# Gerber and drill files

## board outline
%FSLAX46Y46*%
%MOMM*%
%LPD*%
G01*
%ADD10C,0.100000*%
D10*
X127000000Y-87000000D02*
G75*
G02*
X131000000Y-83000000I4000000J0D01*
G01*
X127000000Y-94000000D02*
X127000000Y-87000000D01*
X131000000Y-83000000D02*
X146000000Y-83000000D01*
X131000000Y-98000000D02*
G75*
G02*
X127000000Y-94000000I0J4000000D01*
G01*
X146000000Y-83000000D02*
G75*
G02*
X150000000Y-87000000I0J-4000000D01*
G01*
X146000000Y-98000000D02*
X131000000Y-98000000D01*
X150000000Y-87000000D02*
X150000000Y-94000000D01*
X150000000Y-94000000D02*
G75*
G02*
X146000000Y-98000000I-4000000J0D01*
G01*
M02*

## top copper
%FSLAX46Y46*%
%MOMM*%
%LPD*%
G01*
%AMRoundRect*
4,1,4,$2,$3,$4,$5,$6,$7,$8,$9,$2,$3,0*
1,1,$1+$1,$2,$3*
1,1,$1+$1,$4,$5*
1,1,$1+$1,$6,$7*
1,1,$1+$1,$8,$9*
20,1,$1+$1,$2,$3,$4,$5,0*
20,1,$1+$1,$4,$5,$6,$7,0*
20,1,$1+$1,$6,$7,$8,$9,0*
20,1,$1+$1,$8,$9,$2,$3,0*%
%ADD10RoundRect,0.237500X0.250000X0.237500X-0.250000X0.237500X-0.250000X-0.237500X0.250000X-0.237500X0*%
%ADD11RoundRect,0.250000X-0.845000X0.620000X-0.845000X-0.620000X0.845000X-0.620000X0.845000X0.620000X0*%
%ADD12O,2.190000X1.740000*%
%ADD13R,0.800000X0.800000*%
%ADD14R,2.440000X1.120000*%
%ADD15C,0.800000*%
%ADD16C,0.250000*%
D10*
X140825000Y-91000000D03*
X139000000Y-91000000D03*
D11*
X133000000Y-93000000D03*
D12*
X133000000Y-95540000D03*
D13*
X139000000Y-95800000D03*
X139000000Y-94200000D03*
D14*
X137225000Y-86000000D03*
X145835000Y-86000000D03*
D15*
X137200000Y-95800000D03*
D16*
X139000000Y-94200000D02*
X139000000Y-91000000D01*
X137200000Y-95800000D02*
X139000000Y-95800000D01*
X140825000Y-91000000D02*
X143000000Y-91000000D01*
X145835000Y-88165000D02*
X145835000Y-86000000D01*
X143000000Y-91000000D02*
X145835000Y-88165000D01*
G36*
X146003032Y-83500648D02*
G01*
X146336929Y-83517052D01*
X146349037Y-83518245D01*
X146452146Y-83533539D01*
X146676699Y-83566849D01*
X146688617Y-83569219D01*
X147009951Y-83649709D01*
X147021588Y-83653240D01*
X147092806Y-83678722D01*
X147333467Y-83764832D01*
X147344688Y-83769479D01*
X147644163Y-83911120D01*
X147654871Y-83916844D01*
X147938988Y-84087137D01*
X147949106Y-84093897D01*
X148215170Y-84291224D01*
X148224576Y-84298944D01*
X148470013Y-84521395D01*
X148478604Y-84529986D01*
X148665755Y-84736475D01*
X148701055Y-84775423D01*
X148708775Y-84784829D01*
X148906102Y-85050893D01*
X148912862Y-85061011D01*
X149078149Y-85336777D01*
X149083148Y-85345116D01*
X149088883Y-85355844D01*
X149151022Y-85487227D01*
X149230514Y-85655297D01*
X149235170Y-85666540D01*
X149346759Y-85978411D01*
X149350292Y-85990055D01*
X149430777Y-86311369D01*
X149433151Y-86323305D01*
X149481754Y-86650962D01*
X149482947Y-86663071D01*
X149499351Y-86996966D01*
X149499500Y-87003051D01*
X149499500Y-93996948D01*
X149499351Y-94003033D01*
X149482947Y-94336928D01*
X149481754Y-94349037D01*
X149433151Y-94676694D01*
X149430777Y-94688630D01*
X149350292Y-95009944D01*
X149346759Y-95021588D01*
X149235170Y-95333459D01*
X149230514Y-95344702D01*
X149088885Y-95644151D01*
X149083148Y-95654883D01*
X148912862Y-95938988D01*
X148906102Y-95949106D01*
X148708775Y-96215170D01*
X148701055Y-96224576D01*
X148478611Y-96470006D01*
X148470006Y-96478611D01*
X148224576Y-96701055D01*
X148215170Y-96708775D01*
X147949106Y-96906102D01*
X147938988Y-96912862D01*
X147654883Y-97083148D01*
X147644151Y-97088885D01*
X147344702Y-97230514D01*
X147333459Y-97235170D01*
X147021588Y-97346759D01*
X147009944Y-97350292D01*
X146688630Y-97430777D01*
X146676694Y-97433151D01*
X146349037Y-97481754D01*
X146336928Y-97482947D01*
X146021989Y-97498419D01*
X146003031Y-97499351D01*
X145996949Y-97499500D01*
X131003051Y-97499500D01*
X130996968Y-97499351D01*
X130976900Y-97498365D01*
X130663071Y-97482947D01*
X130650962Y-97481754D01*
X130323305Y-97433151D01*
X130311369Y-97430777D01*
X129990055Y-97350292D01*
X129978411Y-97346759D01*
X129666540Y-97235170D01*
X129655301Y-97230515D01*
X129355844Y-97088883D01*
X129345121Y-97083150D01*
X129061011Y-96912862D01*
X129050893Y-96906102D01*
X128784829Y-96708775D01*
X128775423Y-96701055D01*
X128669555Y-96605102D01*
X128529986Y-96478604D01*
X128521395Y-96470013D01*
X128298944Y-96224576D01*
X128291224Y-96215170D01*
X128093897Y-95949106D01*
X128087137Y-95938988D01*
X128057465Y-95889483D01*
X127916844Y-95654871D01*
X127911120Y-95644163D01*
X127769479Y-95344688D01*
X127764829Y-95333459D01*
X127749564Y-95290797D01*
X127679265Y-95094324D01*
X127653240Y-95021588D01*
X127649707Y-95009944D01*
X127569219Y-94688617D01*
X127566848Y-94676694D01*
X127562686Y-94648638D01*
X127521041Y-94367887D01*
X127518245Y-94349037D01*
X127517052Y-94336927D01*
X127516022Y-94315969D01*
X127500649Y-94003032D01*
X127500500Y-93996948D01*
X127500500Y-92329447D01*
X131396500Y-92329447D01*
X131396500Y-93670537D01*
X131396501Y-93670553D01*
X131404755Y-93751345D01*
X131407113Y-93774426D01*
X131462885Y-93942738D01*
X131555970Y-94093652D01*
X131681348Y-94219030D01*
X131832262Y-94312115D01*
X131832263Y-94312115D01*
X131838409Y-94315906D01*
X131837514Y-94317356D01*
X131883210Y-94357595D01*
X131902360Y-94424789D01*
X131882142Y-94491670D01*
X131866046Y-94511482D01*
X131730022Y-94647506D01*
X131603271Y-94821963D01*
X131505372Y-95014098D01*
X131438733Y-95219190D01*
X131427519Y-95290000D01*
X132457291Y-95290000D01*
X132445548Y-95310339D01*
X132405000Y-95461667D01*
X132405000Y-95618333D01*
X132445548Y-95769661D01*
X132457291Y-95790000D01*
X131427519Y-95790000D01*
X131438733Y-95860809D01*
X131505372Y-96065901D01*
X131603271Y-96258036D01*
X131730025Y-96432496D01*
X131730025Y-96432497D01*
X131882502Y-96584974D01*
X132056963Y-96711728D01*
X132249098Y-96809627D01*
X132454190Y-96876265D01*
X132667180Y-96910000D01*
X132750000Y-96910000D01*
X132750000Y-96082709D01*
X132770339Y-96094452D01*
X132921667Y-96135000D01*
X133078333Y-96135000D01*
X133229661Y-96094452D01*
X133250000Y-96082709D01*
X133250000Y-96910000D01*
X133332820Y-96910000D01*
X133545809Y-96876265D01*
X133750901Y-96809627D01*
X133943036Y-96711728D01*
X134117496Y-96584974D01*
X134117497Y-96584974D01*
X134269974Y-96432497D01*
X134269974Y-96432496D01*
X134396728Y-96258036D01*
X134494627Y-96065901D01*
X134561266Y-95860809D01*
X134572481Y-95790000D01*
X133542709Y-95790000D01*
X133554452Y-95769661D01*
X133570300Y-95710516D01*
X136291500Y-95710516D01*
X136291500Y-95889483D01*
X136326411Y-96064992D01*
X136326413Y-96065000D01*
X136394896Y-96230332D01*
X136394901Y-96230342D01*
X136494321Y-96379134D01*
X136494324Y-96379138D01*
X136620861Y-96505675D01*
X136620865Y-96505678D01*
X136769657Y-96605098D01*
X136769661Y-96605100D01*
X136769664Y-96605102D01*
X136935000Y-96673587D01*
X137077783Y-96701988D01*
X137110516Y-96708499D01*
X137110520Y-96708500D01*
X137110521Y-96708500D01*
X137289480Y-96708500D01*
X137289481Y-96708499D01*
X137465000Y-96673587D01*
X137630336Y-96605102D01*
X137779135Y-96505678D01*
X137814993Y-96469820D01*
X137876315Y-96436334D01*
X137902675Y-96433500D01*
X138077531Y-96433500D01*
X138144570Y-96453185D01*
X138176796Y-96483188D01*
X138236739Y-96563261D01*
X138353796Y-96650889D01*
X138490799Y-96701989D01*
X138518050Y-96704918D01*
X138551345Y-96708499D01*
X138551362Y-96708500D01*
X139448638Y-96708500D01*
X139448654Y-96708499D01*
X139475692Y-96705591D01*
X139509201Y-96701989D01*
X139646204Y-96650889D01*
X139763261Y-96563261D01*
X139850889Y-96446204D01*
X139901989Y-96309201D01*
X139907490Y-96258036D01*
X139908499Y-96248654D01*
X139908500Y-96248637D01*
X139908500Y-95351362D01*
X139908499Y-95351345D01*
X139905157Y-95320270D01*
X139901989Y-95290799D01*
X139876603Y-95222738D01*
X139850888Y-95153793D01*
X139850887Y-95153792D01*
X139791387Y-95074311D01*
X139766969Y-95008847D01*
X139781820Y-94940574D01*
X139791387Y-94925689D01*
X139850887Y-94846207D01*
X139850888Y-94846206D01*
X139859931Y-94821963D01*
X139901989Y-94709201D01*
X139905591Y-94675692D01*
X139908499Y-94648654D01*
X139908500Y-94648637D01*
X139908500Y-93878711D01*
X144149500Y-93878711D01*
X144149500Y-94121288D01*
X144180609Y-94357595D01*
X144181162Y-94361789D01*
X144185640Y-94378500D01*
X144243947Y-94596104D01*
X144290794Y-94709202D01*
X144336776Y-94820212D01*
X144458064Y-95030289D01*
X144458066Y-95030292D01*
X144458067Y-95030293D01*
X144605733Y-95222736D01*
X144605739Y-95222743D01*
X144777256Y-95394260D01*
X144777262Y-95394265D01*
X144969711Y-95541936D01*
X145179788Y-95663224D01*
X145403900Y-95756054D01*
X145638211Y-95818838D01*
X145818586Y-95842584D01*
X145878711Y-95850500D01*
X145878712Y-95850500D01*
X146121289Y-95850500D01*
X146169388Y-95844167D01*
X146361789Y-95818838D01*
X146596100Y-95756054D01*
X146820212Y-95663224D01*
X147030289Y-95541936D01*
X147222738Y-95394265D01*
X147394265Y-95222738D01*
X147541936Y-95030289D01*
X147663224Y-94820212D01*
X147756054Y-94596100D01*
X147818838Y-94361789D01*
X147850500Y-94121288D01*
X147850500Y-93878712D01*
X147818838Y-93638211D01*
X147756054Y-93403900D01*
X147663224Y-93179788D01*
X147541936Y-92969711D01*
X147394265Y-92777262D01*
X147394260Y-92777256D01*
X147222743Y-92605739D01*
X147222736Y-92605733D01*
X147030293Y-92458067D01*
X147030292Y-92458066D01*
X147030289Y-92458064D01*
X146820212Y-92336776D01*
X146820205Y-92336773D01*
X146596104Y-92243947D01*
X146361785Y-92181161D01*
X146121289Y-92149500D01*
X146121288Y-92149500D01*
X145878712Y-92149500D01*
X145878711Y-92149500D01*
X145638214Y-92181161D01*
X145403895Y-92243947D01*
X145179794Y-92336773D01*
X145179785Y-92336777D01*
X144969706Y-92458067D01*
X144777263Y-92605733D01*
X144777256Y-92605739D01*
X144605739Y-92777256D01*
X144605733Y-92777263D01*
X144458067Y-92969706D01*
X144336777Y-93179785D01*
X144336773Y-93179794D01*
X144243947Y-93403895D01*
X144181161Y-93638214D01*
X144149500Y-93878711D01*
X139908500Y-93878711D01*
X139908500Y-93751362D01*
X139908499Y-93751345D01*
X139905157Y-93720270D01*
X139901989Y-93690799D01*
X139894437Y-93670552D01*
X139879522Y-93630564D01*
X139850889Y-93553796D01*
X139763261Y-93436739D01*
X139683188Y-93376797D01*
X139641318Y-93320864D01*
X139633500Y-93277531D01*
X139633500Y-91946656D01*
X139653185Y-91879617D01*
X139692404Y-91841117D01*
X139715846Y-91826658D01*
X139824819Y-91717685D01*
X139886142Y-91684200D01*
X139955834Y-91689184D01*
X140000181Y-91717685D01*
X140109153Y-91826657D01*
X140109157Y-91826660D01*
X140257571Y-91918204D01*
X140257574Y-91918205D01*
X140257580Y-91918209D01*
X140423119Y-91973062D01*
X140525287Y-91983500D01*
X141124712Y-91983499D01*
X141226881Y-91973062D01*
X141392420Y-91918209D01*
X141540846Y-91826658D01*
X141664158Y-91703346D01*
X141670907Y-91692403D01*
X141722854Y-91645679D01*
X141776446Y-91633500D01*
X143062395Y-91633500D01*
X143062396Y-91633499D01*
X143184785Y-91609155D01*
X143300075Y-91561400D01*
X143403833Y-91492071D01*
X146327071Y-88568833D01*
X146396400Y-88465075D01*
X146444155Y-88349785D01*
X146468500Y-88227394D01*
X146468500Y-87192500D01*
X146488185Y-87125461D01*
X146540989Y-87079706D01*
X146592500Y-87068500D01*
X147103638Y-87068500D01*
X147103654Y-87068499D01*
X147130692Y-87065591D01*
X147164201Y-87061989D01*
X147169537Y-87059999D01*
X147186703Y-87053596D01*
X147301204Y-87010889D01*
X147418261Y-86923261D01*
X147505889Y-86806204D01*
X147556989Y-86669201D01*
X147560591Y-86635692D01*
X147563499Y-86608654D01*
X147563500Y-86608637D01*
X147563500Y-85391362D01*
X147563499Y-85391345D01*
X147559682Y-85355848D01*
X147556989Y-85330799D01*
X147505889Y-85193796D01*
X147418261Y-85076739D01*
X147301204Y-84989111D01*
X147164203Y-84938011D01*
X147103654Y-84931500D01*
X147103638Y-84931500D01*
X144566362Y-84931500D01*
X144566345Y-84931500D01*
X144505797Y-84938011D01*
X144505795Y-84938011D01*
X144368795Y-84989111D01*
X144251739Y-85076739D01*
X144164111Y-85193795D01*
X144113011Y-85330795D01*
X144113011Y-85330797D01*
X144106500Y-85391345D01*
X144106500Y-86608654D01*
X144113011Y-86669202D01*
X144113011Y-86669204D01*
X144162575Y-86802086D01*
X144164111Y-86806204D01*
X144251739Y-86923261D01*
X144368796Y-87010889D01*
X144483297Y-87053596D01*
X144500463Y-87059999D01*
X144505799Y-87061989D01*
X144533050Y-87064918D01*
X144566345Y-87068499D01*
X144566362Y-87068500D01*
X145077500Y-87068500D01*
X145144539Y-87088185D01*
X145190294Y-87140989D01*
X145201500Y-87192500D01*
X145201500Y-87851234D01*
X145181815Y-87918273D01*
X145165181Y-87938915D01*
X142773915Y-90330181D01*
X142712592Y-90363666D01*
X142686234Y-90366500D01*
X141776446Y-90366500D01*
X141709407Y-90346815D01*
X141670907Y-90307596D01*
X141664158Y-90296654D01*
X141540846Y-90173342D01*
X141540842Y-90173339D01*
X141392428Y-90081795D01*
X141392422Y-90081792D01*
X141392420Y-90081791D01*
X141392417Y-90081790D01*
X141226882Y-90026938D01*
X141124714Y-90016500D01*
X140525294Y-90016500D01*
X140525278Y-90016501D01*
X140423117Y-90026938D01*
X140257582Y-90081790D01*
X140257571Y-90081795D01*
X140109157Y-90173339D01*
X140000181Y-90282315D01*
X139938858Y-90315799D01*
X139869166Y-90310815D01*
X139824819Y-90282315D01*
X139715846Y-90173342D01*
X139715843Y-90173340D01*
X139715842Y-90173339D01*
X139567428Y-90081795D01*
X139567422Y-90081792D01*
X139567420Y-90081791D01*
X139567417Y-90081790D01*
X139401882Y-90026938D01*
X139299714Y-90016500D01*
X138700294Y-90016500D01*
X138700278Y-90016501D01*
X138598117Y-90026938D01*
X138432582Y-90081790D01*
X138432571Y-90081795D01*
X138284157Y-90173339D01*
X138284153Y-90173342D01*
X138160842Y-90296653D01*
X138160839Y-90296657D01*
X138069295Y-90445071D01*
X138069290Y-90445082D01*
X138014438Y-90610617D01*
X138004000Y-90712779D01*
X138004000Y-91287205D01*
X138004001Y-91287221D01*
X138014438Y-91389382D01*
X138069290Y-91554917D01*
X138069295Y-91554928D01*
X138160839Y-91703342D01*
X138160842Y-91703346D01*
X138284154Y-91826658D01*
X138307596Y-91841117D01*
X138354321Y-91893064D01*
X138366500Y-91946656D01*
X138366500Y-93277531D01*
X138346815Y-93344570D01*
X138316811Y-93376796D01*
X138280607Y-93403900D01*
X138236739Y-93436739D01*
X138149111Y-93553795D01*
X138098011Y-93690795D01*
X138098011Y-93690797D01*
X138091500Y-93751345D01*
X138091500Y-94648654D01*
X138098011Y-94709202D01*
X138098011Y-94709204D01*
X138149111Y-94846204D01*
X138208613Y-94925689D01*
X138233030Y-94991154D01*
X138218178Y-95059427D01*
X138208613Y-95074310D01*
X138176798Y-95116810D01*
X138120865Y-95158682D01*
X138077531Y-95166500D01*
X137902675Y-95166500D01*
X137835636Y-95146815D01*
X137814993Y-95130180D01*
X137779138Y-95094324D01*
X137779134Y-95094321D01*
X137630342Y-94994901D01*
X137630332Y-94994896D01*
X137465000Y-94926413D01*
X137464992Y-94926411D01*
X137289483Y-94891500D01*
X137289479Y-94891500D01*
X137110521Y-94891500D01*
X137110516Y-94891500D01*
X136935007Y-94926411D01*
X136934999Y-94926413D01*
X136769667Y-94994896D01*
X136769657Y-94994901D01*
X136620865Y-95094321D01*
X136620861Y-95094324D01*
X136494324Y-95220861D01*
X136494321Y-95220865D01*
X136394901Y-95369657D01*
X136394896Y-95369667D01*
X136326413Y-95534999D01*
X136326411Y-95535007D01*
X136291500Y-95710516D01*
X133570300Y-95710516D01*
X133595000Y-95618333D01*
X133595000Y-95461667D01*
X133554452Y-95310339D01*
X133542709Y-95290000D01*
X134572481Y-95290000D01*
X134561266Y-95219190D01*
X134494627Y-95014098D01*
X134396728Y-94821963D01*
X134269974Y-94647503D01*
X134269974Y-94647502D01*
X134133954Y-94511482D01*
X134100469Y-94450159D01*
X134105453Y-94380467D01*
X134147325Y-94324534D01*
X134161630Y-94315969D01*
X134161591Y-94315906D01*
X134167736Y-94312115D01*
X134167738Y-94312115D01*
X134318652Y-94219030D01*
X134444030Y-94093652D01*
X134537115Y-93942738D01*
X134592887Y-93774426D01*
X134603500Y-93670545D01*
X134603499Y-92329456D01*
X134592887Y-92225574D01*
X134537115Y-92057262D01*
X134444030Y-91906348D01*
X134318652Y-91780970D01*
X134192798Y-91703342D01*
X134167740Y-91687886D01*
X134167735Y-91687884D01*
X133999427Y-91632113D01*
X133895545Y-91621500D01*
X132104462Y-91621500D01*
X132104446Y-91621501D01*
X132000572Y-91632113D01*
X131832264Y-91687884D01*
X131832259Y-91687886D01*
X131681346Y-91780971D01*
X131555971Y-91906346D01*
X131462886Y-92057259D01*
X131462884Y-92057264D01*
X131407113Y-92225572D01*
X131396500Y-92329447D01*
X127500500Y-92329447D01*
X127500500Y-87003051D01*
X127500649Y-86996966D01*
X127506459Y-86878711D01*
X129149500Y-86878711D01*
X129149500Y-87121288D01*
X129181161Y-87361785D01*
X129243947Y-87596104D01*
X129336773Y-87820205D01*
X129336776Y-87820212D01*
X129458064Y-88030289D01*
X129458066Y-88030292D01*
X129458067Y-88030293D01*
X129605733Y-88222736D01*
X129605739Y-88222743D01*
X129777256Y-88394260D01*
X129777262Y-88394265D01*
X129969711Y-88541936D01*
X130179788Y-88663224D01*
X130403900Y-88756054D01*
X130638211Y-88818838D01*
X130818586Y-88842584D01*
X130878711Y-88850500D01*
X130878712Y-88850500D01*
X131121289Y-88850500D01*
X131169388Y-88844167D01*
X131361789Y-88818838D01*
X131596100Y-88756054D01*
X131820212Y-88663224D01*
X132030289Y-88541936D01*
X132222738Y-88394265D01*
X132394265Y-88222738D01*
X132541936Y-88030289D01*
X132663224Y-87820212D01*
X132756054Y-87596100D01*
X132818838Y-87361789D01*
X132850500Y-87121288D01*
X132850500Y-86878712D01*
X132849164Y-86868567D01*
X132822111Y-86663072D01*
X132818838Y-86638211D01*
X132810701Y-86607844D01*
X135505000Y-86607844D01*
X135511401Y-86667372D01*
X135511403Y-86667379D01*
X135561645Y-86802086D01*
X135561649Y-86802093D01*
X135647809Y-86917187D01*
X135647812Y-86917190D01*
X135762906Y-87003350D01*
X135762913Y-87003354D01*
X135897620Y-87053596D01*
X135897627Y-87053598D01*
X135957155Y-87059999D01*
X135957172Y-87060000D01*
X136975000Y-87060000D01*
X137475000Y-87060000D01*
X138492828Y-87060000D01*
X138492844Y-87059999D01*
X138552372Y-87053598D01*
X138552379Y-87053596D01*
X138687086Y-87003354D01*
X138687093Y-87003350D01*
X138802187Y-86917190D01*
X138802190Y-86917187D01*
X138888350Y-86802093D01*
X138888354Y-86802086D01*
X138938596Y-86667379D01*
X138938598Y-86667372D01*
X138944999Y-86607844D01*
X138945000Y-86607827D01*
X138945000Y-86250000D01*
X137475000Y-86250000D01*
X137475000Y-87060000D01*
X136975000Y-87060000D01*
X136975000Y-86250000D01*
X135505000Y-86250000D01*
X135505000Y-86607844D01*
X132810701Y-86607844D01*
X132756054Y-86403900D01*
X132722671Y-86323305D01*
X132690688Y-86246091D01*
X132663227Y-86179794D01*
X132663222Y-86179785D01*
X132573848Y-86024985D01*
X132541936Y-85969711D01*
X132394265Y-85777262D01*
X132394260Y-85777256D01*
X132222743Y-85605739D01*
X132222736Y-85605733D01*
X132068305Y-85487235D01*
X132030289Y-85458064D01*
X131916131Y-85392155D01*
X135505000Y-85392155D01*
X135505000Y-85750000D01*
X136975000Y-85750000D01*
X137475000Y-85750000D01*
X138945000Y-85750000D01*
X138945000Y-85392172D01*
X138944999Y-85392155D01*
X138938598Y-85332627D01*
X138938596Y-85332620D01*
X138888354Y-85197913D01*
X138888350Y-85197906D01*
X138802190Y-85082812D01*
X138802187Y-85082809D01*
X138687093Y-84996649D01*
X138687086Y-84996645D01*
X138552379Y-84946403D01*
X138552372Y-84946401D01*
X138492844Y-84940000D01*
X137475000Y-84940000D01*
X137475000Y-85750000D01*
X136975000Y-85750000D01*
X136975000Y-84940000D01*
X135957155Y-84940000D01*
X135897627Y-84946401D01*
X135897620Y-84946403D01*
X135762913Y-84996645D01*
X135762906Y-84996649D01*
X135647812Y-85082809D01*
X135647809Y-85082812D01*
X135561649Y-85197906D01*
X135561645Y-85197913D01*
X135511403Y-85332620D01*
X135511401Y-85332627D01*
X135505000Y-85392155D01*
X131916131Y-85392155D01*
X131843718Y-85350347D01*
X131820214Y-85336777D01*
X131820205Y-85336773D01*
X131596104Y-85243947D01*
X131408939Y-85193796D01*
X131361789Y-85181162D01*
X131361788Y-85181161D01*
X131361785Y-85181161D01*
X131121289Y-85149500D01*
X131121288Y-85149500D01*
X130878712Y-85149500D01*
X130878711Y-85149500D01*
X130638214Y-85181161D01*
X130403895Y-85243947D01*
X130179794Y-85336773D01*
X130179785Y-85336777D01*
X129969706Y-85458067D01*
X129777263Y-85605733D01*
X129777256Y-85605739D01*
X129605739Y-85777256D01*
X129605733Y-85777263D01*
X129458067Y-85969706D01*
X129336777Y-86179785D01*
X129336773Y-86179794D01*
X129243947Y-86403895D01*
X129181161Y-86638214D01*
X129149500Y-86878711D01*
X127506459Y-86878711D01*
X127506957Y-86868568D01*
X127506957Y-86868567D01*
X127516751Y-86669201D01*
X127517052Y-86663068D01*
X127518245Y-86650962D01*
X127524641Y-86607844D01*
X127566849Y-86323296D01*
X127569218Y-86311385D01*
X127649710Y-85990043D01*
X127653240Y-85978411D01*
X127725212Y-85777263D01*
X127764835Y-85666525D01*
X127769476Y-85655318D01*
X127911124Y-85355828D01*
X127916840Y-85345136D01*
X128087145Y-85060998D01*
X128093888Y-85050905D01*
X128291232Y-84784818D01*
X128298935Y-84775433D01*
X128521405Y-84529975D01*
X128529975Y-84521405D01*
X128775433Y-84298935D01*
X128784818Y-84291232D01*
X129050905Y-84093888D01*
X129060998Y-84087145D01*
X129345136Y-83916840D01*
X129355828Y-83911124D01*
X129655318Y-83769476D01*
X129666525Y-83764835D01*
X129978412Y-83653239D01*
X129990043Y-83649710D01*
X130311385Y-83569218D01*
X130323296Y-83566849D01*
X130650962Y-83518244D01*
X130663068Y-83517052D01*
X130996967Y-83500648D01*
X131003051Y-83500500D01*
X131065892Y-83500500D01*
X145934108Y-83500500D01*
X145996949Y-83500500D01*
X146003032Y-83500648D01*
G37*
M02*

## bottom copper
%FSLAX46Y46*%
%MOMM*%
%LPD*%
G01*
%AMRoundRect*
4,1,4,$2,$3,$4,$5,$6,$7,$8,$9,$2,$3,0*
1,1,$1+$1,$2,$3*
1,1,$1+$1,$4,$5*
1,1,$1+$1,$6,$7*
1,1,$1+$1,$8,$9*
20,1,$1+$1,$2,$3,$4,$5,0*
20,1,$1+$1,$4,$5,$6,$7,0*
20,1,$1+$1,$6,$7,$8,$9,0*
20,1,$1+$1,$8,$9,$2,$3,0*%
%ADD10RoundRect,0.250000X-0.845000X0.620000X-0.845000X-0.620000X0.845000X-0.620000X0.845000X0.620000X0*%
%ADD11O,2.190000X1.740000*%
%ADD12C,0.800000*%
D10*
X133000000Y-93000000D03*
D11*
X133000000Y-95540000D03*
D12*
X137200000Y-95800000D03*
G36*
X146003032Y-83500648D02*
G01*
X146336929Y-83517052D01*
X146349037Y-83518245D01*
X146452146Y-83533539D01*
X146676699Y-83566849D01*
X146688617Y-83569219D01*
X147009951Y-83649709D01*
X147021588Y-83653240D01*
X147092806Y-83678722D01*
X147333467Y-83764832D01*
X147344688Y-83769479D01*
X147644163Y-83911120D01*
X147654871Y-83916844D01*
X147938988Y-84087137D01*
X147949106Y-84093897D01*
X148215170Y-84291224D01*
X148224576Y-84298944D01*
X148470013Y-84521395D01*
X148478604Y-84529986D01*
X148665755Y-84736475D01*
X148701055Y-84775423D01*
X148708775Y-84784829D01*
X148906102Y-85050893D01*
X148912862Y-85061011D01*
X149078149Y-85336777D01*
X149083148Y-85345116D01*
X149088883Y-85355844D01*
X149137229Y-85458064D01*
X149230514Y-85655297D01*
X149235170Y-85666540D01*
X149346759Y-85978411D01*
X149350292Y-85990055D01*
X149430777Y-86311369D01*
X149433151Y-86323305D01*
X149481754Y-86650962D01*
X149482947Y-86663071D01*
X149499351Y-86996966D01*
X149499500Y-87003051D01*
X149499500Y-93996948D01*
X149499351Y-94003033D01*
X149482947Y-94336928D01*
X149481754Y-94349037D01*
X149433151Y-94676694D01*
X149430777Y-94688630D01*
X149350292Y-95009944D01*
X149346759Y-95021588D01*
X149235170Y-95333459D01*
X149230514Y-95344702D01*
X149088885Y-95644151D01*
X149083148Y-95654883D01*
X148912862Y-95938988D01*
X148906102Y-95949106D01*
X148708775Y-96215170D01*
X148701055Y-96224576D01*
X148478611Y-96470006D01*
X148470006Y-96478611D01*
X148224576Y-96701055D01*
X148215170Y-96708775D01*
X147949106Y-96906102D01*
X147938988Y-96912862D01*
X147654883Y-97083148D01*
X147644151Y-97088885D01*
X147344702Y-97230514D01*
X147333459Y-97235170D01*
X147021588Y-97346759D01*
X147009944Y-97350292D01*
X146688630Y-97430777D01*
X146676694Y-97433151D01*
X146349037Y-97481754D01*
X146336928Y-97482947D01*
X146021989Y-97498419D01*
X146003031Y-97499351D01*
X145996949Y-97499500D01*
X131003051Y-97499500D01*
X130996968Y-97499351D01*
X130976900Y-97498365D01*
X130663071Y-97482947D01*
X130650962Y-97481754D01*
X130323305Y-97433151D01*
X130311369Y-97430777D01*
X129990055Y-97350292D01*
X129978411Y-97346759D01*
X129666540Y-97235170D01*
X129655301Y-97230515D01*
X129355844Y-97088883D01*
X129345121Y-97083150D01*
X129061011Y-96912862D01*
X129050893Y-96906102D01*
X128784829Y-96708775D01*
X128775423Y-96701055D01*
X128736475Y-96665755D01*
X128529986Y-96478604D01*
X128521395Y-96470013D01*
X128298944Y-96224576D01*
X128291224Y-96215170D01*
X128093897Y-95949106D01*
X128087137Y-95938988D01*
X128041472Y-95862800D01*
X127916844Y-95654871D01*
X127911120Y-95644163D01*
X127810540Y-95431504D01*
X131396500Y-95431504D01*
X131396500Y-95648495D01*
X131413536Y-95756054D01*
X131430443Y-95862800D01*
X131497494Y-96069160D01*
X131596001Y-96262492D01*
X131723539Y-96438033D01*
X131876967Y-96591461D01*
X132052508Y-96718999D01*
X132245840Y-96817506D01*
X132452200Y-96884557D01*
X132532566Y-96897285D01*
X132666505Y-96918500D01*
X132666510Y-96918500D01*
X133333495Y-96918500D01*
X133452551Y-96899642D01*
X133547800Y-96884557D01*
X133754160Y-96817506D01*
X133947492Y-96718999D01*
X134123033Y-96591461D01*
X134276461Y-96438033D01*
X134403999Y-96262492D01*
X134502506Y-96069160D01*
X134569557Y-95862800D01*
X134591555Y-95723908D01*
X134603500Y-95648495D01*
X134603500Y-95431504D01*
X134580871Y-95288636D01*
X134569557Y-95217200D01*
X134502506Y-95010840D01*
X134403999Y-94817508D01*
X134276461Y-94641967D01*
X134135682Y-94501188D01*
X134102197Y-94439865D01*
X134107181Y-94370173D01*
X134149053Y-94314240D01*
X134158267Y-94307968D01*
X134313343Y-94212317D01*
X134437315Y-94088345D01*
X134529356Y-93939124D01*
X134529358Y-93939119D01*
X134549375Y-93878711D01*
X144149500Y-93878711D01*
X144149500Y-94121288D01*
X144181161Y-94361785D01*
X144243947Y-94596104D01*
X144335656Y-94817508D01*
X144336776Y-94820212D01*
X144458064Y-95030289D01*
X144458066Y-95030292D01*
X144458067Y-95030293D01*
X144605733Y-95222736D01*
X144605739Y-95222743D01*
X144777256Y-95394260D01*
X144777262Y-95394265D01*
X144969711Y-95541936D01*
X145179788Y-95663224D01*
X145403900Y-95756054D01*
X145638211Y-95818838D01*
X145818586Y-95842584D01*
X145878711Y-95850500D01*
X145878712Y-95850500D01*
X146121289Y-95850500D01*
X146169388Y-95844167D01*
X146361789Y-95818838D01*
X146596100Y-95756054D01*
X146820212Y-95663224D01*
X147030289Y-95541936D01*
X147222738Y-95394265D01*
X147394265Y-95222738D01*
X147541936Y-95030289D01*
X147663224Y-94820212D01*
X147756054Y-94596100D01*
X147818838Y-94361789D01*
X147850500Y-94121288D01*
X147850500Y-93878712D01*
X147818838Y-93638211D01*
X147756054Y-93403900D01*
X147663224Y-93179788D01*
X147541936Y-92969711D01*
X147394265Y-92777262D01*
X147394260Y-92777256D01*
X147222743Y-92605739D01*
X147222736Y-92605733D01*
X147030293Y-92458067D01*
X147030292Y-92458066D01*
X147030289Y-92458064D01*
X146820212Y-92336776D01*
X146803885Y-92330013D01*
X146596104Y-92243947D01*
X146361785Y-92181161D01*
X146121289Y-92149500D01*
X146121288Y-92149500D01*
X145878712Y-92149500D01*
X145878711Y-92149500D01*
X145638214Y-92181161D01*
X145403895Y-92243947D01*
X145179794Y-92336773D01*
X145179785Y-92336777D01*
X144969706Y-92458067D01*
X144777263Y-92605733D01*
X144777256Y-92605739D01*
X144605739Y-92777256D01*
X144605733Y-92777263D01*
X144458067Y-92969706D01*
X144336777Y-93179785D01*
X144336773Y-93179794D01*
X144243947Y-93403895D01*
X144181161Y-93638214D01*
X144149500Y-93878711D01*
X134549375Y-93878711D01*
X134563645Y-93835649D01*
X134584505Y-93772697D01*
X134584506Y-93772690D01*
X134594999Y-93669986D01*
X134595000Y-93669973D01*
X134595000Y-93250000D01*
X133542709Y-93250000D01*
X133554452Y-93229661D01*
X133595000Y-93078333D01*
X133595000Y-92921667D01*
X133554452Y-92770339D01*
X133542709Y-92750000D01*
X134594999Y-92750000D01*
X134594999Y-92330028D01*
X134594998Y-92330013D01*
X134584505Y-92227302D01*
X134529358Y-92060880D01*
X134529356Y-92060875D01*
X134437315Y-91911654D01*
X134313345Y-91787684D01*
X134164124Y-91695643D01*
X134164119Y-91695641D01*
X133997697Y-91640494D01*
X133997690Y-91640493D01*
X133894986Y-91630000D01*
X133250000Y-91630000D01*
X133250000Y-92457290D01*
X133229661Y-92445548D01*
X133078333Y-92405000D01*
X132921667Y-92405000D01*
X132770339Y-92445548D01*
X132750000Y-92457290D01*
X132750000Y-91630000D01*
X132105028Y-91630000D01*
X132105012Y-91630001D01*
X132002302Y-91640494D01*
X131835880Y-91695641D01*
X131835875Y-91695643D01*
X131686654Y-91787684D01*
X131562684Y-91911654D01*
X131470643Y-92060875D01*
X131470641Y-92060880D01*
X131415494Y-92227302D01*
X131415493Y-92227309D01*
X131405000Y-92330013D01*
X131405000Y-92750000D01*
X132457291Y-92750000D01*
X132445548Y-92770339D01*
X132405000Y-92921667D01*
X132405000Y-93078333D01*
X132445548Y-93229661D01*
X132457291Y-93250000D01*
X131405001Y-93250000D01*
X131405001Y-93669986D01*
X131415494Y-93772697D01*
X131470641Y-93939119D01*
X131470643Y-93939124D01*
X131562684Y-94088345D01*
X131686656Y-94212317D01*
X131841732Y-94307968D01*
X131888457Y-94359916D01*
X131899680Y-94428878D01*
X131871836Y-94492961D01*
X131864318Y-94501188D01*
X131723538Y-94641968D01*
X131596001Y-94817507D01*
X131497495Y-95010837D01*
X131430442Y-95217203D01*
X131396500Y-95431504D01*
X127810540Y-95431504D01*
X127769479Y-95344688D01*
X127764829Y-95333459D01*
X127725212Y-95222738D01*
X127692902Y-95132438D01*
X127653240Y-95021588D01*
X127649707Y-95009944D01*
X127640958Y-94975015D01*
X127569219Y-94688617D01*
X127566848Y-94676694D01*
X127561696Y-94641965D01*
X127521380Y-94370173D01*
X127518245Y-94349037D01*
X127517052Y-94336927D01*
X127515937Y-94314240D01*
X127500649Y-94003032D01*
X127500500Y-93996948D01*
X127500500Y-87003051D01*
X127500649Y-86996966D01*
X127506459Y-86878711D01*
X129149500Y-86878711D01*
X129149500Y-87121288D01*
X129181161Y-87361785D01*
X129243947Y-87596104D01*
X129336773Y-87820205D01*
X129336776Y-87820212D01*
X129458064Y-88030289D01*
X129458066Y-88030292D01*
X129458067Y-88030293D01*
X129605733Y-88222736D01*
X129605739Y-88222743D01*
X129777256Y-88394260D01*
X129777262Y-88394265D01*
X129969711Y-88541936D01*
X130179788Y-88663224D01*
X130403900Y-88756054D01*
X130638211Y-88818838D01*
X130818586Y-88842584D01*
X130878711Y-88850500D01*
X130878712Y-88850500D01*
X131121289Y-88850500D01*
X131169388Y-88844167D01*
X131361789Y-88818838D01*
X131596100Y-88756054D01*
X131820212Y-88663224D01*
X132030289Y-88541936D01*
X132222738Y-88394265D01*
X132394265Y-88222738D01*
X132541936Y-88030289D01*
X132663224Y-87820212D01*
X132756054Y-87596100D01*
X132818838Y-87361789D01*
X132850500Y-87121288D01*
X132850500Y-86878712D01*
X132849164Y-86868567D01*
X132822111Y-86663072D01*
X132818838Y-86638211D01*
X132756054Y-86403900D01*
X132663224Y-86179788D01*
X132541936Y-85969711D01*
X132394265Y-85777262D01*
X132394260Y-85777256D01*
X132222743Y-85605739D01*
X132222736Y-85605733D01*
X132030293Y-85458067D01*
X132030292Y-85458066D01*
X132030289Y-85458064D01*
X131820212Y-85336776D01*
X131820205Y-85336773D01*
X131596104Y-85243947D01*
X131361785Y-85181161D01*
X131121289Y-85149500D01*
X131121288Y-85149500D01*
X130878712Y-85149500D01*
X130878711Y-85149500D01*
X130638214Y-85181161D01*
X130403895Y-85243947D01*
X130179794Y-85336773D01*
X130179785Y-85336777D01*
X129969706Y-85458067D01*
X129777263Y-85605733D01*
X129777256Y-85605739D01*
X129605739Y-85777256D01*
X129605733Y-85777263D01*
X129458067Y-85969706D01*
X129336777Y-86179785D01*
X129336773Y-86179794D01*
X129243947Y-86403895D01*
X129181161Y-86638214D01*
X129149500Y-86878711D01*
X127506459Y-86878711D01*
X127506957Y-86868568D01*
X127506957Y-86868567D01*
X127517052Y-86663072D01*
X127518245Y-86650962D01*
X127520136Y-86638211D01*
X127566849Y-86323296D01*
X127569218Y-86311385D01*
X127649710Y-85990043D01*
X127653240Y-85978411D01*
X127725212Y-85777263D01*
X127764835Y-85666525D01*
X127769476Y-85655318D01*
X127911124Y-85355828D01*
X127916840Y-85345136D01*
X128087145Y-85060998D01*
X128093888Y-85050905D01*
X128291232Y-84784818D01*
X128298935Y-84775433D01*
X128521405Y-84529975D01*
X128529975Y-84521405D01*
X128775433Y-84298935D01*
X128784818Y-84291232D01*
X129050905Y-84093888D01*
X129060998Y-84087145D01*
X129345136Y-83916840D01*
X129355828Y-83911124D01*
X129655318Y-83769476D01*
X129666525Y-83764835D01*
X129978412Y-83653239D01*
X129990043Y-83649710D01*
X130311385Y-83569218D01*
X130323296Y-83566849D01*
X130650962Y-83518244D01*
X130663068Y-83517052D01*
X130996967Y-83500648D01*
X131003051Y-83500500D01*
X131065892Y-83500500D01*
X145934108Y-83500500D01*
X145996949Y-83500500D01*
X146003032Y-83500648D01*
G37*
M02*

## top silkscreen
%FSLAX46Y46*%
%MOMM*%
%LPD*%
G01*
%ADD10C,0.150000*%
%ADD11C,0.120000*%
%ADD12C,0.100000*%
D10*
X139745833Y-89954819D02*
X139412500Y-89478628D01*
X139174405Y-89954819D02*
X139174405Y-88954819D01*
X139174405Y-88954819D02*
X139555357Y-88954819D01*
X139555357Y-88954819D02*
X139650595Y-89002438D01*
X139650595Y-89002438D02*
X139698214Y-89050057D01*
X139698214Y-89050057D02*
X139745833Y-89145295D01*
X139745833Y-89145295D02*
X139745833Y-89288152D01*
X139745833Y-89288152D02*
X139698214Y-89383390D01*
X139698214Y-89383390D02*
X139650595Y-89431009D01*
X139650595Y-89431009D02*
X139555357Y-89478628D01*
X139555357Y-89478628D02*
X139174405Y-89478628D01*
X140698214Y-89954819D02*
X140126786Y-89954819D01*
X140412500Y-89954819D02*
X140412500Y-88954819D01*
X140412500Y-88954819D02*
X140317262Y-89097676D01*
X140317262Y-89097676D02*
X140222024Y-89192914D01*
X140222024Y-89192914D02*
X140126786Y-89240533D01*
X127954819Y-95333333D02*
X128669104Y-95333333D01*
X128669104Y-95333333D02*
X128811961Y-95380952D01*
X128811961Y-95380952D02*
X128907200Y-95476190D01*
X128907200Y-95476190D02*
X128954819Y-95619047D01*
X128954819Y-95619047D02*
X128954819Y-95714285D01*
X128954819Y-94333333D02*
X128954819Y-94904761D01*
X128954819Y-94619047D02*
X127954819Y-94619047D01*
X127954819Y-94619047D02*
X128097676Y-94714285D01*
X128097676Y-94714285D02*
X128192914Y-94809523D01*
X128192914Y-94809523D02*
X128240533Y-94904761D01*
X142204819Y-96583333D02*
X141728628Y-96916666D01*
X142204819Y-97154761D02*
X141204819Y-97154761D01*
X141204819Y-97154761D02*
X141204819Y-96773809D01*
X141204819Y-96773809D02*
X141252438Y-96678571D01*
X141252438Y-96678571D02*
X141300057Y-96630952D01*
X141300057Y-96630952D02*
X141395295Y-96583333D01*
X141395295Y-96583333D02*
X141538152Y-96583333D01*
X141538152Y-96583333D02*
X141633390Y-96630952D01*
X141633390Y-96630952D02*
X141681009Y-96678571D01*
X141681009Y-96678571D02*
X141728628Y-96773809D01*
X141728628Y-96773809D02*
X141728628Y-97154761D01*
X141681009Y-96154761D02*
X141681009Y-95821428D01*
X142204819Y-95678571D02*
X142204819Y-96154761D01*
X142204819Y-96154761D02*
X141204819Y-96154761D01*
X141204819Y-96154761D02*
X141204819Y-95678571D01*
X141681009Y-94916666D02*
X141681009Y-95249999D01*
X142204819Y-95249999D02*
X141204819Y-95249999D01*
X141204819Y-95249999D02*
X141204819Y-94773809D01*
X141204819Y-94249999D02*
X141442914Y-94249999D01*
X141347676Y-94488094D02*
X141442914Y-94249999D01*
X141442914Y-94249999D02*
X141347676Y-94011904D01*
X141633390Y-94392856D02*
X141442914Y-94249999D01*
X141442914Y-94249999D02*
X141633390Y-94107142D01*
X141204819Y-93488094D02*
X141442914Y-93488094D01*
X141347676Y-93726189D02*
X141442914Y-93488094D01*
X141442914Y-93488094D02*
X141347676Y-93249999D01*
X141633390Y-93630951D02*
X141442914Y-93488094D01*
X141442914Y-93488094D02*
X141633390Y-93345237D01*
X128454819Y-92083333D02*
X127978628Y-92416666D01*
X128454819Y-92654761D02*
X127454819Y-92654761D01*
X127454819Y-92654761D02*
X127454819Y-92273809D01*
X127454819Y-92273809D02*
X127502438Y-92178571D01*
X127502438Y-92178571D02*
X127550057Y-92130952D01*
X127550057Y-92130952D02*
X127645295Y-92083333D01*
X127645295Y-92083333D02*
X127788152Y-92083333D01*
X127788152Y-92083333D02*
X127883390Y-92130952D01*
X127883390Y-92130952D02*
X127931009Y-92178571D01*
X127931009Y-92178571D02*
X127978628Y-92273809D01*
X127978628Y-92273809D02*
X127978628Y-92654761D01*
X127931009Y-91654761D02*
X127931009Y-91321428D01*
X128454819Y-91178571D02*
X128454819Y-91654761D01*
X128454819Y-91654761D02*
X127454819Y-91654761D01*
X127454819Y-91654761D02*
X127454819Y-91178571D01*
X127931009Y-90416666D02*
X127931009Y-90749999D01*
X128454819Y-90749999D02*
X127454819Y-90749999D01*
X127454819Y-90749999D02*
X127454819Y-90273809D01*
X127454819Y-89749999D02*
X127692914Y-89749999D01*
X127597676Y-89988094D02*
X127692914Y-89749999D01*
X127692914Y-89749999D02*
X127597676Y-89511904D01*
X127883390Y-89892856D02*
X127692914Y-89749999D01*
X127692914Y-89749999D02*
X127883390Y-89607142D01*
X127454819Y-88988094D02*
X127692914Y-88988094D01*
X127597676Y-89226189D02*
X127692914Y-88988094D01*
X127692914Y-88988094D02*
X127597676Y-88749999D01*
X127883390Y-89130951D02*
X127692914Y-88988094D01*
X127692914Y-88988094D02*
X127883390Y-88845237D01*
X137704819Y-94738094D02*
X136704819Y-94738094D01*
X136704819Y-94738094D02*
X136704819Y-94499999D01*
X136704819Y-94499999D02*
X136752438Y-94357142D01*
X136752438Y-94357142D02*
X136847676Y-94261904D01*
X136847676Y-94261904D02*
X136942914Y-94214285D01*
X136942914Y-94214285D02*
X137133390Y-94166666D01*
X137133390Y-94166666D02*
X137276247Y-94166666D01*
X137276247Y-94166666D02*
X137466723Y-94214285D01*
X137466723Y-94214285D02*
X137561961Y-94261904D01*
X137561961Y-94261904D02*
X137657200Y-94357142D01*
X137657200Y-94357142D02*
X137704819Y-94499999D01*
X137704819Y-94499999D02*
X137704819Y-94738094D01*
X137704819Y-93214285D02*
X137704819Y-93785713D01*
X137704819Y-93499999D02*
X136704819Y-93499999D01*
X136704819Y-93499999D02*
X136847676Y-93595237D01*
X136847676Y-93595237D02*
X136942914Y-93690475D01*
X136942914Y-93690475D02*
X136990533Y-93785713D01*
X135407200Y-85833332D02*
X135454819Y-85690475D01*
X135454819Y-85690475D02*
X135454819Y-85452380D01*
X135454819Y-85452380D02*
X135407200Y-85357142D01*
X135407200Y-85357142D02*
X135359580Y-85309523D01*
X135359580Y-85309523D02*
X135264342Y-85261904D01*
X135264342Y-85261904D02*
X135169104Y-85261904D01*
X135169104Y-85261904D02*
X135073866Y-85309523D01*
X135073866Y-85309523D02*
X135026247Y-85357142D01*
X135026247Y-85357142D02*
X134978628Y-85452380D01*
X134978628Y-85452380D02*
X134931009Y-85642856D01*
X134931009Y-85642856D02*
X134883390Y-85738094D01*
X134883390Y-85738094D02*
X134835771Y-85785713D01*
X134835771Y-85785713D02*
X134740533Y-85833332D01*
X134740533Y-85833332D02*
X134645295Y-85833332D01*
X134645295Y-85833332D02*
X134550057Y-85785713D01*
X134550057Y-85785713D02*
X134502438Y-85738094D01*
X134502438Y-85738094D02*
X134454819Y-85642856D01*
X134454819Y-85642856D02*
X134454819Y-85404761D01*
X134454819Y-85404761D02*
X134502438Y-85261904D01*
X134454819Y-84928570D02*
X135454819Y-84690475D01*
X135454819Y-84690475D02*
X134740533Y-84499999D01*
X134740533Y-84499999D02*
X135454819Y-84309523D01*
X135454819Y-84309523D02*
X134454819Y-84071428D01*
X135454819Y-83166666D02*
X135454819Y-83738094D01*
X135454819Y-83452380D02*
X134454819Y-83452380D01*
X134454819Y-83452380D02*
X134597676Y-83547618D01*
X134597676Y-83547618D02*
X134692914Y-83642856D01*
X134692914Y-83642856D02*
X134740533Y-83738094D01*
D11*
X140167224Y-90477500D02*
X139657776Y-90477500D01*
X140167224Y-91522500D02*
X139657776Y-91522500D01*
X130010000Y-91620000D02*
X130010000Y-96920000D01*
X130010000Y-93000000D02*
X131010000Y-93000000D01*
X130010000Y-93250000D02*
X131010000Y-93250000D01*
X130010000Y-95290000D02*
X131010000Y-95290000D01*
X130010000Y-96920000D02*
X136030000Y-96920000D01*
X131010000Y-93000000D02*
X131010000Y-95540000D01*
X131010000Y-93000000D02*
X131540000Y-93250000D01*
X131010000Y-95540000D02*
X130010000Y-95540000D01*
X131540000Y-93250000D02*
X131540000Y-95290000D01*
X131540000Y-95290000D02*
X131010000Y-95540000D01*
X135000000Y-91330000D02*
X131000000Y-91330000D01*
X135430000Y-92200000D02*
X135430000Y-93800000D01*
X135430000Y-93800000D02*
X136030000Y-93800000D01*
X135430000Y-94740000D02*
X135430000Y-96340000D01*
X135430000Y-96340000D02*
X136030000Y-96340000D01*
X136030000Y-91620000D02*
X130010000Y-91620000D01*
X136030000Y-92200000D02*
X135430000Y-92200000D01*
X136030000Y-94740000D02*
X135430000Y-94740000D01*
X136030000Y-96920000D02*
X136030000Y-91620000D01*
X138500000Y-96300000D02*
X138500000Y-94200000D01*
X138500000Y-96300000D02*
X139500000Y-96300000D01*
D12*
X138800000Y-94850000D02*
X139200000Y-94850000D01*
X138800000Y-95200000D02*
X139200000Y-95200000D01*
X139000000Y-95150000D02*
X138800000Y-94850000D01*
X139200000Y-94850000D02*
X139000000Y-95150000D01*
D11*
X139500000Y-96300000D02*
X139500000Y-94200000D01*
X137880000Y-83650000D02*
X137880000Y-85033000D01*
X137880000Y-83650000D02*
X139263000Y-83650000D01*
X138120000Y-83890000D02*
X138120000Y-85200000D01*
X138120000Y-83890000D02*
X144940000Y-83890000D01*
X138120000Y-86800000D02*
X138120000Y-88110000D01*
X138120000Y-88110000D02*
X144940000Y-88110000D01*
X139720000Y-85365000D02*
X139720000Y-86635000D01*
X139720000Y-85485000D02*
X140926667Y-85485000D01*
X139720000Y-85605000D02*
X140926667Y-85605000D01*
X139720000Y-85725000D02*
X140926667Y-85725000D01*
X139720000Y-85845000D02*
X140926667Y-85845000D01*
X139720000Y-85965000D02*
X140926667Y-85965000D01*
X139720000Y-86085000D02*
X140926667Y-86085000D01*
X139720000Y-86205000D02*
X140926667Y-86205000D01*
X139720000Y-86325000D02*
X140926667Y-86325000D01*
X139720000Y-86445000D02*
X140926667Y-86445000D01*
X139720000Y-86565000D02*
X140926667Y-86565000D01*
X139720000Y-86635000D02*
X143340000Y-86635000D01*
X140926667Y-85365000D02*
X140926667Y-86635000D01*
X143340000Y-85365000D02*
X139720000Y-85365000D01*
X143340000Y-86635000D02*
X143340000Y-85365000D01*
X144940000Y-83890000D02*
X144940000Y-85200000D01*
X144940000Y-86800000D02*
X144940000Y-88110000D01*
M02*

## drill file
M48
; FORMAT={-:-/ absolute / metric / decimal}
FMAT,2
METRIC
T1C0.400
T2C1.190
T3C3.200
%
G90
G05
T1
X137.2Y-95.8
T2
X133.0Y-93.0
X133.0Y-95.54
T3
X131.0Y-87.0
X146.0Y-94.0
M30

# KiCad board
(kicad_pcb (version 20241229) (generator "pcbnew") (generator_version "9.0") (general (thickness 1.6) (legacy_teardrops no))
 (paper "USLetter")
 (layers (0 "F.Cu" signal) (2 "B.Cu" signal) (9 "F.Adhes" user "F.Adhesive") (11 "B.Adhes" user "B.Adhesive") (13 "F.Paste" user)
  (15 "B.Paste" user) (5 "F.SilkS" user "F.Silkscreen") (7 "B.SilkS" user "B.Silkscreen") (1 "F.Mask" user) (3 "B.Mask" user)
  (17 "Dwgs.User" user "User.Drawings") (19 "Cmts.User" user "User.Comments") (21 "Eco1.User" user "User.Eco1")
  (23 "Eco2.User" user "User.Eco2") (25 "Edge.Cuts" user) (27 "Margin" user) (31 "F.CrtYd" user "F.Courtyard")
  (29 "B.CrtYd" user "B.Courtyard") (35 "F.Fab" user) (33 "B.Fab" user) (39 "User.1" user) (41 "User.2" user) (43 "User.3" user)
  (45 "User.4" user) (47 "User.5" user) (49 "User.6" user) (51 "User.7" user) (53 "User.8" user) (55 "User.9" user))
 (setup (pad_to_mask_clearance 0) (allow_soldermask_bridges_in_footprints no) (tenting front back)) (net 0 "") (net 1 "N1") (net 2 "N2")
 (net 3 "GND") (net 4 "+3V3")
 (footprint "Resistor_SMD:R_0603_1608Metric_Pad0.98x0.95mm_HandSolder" (layer "F.Cu") (at 139.9125 91 180)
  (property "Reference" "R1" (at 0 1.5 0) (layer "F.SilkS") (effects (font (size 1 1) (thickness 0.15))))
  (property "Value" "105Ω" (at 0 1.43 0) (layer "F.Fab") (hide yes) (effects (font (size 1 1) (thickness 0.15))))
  (fp_line (start -0.254724 0.5225) (end 0.254724 0.5225) (stroke (width 0.12) (type solid)) (layer "F.SilkS"))
  (fp_line (start -0.254724 -0.5225) (end 0.254724 -0.5225) (stroke (width 0.12) (type solid)) (layer "F.SilkS"))
  (pad "1" smd roundrect (at -0.9125 0 180) (size 0.975 0.95) (layers "F.Cu" "F.Mask" "F.Paste") (roundrect_rratio 0.25) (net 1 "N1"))
  (pad "2" smd roundrect (at 0.9125 0 180) (size 0.975 0.95) (layers "F.Cu" "F.Mask" "F.Paste") (roundrect_rratio 0.25) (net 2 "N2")))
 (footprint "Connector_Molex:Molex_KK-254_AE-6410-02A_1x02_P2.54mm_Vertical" (layer "F.Cu") (at 133 93 -90)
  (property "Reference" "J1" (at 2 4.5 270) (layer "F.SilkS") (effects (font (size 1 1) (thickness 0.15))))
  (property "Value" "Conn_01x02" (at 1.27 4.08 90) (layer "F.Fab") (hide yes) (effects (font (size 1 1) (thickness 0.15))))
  (fp_line (start -1.38 2.99) (end 3.92 2.99) (stroke (width 0.12) (type solid)) (layer "F.SilkS"))
  (fp_line (start 0 2.99) (end 0 1.99) (stroke (width 0.12) (type solid)) (layer "F.SilkS"))
  (fp_line (start 0.25 2.99) (end 0.25 1.99) (stroke (width 0.12) (type solid)) (layer "F.SilkS"))
  (fp_line (start 2.29 2.99) (end 2.29 1.99) (stroke (width 0.12) (type solid)) (layer "F.SilkS"))
  (fp_line (start 3.92 2.99) (end 3.92 -3.03) (stroke (width 0.12) (type solid)) (layer "F.SilkS"))
  (fp_line (start 0 1.99) (end 2.54 1.99) (stroke (width 0.12) (type solid)) (layer "F.SilkS"))
  (fp_line (start 0 1.99) (end 0.25 1.46) (stroke (width 0.12) (type solid)) (layer "F.SilkS"))
  (fp_line (start 2.54 1.99) (end 2.54 2.99) (stroke (width 0.12) (type solid)) (layer "F.SilkS"))
  (fp_line (start 0.25 1.46) (end 2.29 1.46) (stroke (width 0.12) (type solid)) (layer "F.SilkS"))
  (fp_line (start 2.29 1.46) (end 2.54 1.99) (stroke (width 0.12) (type solid)) (layer "F.SilkS"))
  (fp_line (start -1.67 -2) (end -1.67 2) (stroke (width 0.12) (type solid)) (layer "F.SilkS"))
  (fp_line (start -0.8 -2.43) (end 0.8 -2.43) (stroke (width 0.12) (type solid)) (layer "F.SilkS"))
  (fp_line (start 0.8 -2.43) (end 0.8 -3.03) (stroke (width 0.12) (type solid)) (layer "F.SilkS"))
  (fp_line (start 1.74 -2.43) (end 3.34 -2.43) (stroke (width 0.12) (type solid)) (layer "F.SilkS"))
  (fp_line (start 3.34 -2.43) (end 3.34 -3.03) (stroke (width 0.12) (type solid)) (layer "F.SilkS"))
  (fp_line (start -1.38 -3.03) (end -1.38 2.99) (stroke (width 0.12) (type solid)) (layer "F.SilkS"))
  (fp_line (start -0.8 -3.03) (end -0.8 -2.43) (stroke (width 0.12) (type solid)) (layer "F.SilkS"))
  (fp_line (start 1.74 -3.03) (end 1.74 -2.43) (stroke (width 0.12) (type solid)) (layer "F.SilkS"))
  (fp_line (start 3.92 -3.03) (end -1.38 -3.03) (stroke (width 0.12) (type solid)) (layer "F.SilkS"))
  (pad "1" thru_hole roundrect (at 0 0 270) (size 1.74 2.19) (drill 1.19) (layers "*.Cu" "*.Mask") (remove_unused_layers no)
   (roundrect_rratio 0.143678) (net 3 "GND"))
  (pad "2" thru_hole oval (at 2.54 0 270) (size 1.74 2.19) (drill 1.19) (layers "*.Cu" "*.Mask") (remove_unused_layers no) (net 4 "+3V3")))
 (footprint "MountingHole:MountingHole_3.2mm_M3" (layer "F.Cu") (at 146 94)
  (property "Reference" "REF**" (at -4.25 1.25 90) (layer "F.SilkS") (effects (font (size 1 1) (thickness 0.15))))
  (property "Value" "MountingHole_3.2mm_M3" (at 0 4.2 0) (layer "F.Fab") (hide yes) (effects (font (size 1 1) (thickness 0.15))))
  (pad "" np_thru_hole circle (at 0 0) (size 3.2 3.2) (drill 3.2) (layers "*.Cu" "*.Mask")))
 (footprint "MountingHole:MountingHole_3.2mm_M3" (layer "F.Cu") (at 131 87)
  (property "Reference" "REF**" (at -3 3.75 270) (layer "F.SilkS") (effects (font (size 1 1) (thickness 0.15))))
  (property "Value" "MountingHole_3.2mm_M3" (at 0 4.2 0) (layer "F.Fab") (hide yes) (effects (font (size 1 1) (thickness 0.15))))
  (pad "" np_thru_hole circle (at 0 0) (size 3.2 3.2) (drill 3.2) (layers "*.Cu" "*.Mask")))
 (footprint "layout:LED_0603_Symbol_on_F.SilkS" (layer "F.Cu") (at 139 95 90)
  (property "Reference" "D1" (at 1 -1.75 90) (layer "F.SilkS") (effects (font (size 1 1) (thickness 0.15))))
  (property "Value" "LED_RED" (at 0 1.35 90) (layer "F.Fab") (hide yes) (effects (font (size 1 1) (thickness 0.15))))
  (fp_line (start -1.3 -0.5) (end 0.8 -0.5) (stroke (width 0.12) (type solid)) (layer "F.SilkS"))
  (fp_line (start -1.3 -0.5) (end -1.3 0.5) (stroke (width 0.12) (type solid)) (layer "F.SilkS"))
  (fp_line (start 0.15 -0.2) (end 0.15 0.2) (stroke (width 0.1) (type solid)) (layer "F.SilkS"))
  (fp_line (start -0.2 -0.2) (end -0.2 0.2) (stroke (width 0.1) (type solid)) (layer "F.SilkS"))
  (fp_line (start -0.15 0) (end 0.15 -0.2) (stroke (width 0.1) (type solid)) (layer "F.SilkS"))
  (fp_line (start 0.15 0.2) (end -0.15 0) (stroke (width 0.1) (type solid)) (layer "F.SilkS"))
  (fp_line (start -1.3 0.5) (end 0.8 0.5) (stroke (width 0.12) (type solid)) (layer "F.SilkS"))
  (pad "1" smd rect (at -0.8 0 270) (size 0.8 0.8) (layers "F.Cu" "F.Mask" "F.Paste") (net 3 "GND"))
  (pad "2" smd rect (at 0.8 0 270) (size 0.8 0.8) (layers "F.Cu" "F.Mask" "F.Paste") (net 2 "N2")))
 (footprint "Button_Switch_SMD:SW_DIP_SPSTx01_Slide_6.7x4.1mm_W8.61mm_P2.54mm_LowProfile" (layer "F.Cu") (at 141.53 86)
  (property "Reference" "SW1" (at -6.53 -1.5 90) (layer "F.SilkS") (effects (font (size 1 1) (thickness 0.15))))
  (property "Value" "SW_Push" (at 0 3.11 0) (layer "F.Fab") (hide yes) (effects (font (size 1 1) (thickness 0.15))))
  (fp_line (start -3.65 -2.35) (end -3.65 -0.967) (stroke (width 0.12) (type solid)) (layer "F.SilkS"))
  (fp_line (start -3.65 -2.35) (end -2.267 -2.35) (stroke (width 0.12) (type solid)) (layer "F.SilkS"))
  (fp_line (start -3.41 -2.11) (end -3.41 -0.8) (stroke (width 0.12) (type solid)) (layer "F.SilkS"))
  (fp_line (start -3.41 -2.11) (end 3.41 -2.11) (stroke (width 0.12) (type solid)) (layer "F.SilkS"))
  (fp_line (start -3.41 0.8) (end -3.41 2.11) (stroke (width 0.12) (type solid)) (layer "F.SilkS"))
  (fp_line (start -3.41 2.11) (end 3.41 2.11) (stroke (width 0.12) (type solid)) (layer "F.SilkS"))
  (fp_line (start -1.81 -0.635) (end -1.81 0.635) (stroke (width 0.12) (type solid)) (layer "F.SilkS"))
  (fp_line (start -1.81 -0.515) (end -0.603333 -0.515) (stroke (width 0.12) (type solid)) (layer "F.SilkS"))
  (fp_line (start -1.81 -0.395) (end -0.603333 -0.395) (stroke (width 0.12) (type solid)) (layer "F.SilkS"))
  (fp_line (start -1.81 -0.275) (end -0.603333 -0.275) (stroke (width 0.12) (type solid)) (layer "F.SilkS"))
  (fp_line (start -1.81 -0.155) (end -0.603333 -0.155) (stroke (width 0.12) (type solid)) (layer "F.SilkS"))
  (fp_line (start -1.81 -0.035) (end -0.603333 -0.035) (stroke (width 0.12) (type solid)) (layer "F.SilkS"))
  (fp_line (start -1.81 0.085) (end -0.603333 0.085) (stroke (width 0.12) (type solid)) (layer "F.SilkS"))
  (fp_line (start -1.81 0.205) (end -0.603333 0.205) (stroke (width 0.12) (type solid)) (layer "F.SilkS"))
  (fp_line (start -1.81 0.325) (end -0.603333 0.325) (stroke (width 0.12) (type solid)) (layer "F.SilkS"))
  (fp_line (start -1.81 0.445) (end -0.603333 0.445) (stroke (width 0.12) (type solid)) (layer "F.SilkS"))
  (fp_line (start -1.81 0.565) (end -0.603333 0.565) (stroke (width 0.12) (type solid)) (layer "F.SilkS"))
  (fp_line (start -1.81 0.635) (end 1.81 0.635) (stroke (width 0.12) (type solid)) (layer "F.SilkS"))
  (fp_line (start -0.603333 -0.635) (end -0.603333 0.635) (stroke (width 0.12) (type solid)) (layer "F.SilkS"))
  (fp_line (start 1.81 -0.635) (end -1.81 -0.635) (stroke (width 0.12) (type solid)) (layer "F.SilkS"))
  (fp_line (start 1.81 0.635) (end 1.81 -0.635) (stroke (width 0.12) (type solid)) (layer "F.SilkS"))
  (fp_line (start 3.41 -2.11) (end 3.41 -0.8) (stroke (width 0.12) (type solid)) (layer "F.SilkS"))
  (fp_line (start 3.41 0.8) (end 3.41 2.11) (stroke (width 0.12) (type solid)) (layer "F.SilkS"))
  (pad "1" smd rect (at -4.305 0) (size 2.44 1.12) (layers "F.Cu" "F.Mask" "F.Paste") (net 4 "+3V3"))
  (pad "2" smd rect (at 4.305 0) (size 2.44 1.12) (layers "F.Cu" "F.Mask" "F.Paste") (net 1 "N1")))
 (gr_arc (start 127 87) (mid 128.171573 84.171573) (end 131 83) (stroke (width 0.1) (type default)) (layer "Edge.Cuts"))
 (gr_line (start 127 94) (end 127 87) (stroke (width 0.1) (type default)) (layer "Edge.Cuts"))
 (gr_line (start 131 83) (end 146 83) (stroke (width 0.1) (type default)) (layer "Edge.Cuts"))
 (gr_arc (start 131 98) (mid 128.171573 96.828427) (end 127 94) (stroke (width 0.1) (type default)) (layer "Edge.Cuts"))
 (gr_arc (start 146 83) (mid 148.828427 84.171573) (end 150 87) (stroke (width 0.1) (type default)) (layer "Edge.Cuts"))
 (gr_line (start 146 98) (end 131 98) (stroke (width 0.1) (type default)) (layer "Edge.Cuts"))
 (gr_line (start 150 87) (end 150 94) (stroke (width 0.1) (type default)) (layer "Edge.Cuts"))
 (gr_arc (start 150 94) (mid 148.828427 96.828427) (end 146 98) (stroke (width 0.1) (type default)) (layer "Edge.Cuts"))
 (segment (start 139 94.2) (end 139 91) (width 0.25) (layer "F.Cu") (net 2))
 (segment (start 137.2 95.8) (end 139 95.8) (width 0.25) (layer "F.Cu") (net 3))
 (via (at 137.2 95.8) (size 0.8) (drill 0.4) (layers "F.Cu" "B.Cu") (free yes) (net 3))
 (segment (start 140.825 91) (end 143 91) (width 0.25) (layer "F.Cu") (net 1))
 (segment (start 145.835 88.165) (end 145.835 86) (width 0.25) (layer "F.Cu") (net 1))
 (segment (start 143 91) (end 145.835 88.165) (width 0.25) (layer "F.Cu") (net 1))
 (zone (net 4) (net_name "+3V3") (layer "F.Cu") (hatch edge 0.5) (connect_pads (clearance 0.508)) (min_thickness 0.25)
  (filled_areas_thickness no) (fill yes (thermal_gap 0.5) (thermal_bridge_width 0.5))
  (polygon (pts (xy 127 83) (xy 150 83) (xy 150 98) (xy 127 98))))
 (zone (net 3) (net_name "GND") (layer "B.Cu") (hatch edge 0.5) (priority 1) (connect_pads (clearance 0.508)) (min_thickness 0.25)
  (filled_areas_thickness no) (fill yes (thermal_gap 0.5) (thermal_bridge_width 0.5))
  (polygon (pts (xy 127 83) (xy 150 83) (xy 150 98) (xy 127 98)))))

